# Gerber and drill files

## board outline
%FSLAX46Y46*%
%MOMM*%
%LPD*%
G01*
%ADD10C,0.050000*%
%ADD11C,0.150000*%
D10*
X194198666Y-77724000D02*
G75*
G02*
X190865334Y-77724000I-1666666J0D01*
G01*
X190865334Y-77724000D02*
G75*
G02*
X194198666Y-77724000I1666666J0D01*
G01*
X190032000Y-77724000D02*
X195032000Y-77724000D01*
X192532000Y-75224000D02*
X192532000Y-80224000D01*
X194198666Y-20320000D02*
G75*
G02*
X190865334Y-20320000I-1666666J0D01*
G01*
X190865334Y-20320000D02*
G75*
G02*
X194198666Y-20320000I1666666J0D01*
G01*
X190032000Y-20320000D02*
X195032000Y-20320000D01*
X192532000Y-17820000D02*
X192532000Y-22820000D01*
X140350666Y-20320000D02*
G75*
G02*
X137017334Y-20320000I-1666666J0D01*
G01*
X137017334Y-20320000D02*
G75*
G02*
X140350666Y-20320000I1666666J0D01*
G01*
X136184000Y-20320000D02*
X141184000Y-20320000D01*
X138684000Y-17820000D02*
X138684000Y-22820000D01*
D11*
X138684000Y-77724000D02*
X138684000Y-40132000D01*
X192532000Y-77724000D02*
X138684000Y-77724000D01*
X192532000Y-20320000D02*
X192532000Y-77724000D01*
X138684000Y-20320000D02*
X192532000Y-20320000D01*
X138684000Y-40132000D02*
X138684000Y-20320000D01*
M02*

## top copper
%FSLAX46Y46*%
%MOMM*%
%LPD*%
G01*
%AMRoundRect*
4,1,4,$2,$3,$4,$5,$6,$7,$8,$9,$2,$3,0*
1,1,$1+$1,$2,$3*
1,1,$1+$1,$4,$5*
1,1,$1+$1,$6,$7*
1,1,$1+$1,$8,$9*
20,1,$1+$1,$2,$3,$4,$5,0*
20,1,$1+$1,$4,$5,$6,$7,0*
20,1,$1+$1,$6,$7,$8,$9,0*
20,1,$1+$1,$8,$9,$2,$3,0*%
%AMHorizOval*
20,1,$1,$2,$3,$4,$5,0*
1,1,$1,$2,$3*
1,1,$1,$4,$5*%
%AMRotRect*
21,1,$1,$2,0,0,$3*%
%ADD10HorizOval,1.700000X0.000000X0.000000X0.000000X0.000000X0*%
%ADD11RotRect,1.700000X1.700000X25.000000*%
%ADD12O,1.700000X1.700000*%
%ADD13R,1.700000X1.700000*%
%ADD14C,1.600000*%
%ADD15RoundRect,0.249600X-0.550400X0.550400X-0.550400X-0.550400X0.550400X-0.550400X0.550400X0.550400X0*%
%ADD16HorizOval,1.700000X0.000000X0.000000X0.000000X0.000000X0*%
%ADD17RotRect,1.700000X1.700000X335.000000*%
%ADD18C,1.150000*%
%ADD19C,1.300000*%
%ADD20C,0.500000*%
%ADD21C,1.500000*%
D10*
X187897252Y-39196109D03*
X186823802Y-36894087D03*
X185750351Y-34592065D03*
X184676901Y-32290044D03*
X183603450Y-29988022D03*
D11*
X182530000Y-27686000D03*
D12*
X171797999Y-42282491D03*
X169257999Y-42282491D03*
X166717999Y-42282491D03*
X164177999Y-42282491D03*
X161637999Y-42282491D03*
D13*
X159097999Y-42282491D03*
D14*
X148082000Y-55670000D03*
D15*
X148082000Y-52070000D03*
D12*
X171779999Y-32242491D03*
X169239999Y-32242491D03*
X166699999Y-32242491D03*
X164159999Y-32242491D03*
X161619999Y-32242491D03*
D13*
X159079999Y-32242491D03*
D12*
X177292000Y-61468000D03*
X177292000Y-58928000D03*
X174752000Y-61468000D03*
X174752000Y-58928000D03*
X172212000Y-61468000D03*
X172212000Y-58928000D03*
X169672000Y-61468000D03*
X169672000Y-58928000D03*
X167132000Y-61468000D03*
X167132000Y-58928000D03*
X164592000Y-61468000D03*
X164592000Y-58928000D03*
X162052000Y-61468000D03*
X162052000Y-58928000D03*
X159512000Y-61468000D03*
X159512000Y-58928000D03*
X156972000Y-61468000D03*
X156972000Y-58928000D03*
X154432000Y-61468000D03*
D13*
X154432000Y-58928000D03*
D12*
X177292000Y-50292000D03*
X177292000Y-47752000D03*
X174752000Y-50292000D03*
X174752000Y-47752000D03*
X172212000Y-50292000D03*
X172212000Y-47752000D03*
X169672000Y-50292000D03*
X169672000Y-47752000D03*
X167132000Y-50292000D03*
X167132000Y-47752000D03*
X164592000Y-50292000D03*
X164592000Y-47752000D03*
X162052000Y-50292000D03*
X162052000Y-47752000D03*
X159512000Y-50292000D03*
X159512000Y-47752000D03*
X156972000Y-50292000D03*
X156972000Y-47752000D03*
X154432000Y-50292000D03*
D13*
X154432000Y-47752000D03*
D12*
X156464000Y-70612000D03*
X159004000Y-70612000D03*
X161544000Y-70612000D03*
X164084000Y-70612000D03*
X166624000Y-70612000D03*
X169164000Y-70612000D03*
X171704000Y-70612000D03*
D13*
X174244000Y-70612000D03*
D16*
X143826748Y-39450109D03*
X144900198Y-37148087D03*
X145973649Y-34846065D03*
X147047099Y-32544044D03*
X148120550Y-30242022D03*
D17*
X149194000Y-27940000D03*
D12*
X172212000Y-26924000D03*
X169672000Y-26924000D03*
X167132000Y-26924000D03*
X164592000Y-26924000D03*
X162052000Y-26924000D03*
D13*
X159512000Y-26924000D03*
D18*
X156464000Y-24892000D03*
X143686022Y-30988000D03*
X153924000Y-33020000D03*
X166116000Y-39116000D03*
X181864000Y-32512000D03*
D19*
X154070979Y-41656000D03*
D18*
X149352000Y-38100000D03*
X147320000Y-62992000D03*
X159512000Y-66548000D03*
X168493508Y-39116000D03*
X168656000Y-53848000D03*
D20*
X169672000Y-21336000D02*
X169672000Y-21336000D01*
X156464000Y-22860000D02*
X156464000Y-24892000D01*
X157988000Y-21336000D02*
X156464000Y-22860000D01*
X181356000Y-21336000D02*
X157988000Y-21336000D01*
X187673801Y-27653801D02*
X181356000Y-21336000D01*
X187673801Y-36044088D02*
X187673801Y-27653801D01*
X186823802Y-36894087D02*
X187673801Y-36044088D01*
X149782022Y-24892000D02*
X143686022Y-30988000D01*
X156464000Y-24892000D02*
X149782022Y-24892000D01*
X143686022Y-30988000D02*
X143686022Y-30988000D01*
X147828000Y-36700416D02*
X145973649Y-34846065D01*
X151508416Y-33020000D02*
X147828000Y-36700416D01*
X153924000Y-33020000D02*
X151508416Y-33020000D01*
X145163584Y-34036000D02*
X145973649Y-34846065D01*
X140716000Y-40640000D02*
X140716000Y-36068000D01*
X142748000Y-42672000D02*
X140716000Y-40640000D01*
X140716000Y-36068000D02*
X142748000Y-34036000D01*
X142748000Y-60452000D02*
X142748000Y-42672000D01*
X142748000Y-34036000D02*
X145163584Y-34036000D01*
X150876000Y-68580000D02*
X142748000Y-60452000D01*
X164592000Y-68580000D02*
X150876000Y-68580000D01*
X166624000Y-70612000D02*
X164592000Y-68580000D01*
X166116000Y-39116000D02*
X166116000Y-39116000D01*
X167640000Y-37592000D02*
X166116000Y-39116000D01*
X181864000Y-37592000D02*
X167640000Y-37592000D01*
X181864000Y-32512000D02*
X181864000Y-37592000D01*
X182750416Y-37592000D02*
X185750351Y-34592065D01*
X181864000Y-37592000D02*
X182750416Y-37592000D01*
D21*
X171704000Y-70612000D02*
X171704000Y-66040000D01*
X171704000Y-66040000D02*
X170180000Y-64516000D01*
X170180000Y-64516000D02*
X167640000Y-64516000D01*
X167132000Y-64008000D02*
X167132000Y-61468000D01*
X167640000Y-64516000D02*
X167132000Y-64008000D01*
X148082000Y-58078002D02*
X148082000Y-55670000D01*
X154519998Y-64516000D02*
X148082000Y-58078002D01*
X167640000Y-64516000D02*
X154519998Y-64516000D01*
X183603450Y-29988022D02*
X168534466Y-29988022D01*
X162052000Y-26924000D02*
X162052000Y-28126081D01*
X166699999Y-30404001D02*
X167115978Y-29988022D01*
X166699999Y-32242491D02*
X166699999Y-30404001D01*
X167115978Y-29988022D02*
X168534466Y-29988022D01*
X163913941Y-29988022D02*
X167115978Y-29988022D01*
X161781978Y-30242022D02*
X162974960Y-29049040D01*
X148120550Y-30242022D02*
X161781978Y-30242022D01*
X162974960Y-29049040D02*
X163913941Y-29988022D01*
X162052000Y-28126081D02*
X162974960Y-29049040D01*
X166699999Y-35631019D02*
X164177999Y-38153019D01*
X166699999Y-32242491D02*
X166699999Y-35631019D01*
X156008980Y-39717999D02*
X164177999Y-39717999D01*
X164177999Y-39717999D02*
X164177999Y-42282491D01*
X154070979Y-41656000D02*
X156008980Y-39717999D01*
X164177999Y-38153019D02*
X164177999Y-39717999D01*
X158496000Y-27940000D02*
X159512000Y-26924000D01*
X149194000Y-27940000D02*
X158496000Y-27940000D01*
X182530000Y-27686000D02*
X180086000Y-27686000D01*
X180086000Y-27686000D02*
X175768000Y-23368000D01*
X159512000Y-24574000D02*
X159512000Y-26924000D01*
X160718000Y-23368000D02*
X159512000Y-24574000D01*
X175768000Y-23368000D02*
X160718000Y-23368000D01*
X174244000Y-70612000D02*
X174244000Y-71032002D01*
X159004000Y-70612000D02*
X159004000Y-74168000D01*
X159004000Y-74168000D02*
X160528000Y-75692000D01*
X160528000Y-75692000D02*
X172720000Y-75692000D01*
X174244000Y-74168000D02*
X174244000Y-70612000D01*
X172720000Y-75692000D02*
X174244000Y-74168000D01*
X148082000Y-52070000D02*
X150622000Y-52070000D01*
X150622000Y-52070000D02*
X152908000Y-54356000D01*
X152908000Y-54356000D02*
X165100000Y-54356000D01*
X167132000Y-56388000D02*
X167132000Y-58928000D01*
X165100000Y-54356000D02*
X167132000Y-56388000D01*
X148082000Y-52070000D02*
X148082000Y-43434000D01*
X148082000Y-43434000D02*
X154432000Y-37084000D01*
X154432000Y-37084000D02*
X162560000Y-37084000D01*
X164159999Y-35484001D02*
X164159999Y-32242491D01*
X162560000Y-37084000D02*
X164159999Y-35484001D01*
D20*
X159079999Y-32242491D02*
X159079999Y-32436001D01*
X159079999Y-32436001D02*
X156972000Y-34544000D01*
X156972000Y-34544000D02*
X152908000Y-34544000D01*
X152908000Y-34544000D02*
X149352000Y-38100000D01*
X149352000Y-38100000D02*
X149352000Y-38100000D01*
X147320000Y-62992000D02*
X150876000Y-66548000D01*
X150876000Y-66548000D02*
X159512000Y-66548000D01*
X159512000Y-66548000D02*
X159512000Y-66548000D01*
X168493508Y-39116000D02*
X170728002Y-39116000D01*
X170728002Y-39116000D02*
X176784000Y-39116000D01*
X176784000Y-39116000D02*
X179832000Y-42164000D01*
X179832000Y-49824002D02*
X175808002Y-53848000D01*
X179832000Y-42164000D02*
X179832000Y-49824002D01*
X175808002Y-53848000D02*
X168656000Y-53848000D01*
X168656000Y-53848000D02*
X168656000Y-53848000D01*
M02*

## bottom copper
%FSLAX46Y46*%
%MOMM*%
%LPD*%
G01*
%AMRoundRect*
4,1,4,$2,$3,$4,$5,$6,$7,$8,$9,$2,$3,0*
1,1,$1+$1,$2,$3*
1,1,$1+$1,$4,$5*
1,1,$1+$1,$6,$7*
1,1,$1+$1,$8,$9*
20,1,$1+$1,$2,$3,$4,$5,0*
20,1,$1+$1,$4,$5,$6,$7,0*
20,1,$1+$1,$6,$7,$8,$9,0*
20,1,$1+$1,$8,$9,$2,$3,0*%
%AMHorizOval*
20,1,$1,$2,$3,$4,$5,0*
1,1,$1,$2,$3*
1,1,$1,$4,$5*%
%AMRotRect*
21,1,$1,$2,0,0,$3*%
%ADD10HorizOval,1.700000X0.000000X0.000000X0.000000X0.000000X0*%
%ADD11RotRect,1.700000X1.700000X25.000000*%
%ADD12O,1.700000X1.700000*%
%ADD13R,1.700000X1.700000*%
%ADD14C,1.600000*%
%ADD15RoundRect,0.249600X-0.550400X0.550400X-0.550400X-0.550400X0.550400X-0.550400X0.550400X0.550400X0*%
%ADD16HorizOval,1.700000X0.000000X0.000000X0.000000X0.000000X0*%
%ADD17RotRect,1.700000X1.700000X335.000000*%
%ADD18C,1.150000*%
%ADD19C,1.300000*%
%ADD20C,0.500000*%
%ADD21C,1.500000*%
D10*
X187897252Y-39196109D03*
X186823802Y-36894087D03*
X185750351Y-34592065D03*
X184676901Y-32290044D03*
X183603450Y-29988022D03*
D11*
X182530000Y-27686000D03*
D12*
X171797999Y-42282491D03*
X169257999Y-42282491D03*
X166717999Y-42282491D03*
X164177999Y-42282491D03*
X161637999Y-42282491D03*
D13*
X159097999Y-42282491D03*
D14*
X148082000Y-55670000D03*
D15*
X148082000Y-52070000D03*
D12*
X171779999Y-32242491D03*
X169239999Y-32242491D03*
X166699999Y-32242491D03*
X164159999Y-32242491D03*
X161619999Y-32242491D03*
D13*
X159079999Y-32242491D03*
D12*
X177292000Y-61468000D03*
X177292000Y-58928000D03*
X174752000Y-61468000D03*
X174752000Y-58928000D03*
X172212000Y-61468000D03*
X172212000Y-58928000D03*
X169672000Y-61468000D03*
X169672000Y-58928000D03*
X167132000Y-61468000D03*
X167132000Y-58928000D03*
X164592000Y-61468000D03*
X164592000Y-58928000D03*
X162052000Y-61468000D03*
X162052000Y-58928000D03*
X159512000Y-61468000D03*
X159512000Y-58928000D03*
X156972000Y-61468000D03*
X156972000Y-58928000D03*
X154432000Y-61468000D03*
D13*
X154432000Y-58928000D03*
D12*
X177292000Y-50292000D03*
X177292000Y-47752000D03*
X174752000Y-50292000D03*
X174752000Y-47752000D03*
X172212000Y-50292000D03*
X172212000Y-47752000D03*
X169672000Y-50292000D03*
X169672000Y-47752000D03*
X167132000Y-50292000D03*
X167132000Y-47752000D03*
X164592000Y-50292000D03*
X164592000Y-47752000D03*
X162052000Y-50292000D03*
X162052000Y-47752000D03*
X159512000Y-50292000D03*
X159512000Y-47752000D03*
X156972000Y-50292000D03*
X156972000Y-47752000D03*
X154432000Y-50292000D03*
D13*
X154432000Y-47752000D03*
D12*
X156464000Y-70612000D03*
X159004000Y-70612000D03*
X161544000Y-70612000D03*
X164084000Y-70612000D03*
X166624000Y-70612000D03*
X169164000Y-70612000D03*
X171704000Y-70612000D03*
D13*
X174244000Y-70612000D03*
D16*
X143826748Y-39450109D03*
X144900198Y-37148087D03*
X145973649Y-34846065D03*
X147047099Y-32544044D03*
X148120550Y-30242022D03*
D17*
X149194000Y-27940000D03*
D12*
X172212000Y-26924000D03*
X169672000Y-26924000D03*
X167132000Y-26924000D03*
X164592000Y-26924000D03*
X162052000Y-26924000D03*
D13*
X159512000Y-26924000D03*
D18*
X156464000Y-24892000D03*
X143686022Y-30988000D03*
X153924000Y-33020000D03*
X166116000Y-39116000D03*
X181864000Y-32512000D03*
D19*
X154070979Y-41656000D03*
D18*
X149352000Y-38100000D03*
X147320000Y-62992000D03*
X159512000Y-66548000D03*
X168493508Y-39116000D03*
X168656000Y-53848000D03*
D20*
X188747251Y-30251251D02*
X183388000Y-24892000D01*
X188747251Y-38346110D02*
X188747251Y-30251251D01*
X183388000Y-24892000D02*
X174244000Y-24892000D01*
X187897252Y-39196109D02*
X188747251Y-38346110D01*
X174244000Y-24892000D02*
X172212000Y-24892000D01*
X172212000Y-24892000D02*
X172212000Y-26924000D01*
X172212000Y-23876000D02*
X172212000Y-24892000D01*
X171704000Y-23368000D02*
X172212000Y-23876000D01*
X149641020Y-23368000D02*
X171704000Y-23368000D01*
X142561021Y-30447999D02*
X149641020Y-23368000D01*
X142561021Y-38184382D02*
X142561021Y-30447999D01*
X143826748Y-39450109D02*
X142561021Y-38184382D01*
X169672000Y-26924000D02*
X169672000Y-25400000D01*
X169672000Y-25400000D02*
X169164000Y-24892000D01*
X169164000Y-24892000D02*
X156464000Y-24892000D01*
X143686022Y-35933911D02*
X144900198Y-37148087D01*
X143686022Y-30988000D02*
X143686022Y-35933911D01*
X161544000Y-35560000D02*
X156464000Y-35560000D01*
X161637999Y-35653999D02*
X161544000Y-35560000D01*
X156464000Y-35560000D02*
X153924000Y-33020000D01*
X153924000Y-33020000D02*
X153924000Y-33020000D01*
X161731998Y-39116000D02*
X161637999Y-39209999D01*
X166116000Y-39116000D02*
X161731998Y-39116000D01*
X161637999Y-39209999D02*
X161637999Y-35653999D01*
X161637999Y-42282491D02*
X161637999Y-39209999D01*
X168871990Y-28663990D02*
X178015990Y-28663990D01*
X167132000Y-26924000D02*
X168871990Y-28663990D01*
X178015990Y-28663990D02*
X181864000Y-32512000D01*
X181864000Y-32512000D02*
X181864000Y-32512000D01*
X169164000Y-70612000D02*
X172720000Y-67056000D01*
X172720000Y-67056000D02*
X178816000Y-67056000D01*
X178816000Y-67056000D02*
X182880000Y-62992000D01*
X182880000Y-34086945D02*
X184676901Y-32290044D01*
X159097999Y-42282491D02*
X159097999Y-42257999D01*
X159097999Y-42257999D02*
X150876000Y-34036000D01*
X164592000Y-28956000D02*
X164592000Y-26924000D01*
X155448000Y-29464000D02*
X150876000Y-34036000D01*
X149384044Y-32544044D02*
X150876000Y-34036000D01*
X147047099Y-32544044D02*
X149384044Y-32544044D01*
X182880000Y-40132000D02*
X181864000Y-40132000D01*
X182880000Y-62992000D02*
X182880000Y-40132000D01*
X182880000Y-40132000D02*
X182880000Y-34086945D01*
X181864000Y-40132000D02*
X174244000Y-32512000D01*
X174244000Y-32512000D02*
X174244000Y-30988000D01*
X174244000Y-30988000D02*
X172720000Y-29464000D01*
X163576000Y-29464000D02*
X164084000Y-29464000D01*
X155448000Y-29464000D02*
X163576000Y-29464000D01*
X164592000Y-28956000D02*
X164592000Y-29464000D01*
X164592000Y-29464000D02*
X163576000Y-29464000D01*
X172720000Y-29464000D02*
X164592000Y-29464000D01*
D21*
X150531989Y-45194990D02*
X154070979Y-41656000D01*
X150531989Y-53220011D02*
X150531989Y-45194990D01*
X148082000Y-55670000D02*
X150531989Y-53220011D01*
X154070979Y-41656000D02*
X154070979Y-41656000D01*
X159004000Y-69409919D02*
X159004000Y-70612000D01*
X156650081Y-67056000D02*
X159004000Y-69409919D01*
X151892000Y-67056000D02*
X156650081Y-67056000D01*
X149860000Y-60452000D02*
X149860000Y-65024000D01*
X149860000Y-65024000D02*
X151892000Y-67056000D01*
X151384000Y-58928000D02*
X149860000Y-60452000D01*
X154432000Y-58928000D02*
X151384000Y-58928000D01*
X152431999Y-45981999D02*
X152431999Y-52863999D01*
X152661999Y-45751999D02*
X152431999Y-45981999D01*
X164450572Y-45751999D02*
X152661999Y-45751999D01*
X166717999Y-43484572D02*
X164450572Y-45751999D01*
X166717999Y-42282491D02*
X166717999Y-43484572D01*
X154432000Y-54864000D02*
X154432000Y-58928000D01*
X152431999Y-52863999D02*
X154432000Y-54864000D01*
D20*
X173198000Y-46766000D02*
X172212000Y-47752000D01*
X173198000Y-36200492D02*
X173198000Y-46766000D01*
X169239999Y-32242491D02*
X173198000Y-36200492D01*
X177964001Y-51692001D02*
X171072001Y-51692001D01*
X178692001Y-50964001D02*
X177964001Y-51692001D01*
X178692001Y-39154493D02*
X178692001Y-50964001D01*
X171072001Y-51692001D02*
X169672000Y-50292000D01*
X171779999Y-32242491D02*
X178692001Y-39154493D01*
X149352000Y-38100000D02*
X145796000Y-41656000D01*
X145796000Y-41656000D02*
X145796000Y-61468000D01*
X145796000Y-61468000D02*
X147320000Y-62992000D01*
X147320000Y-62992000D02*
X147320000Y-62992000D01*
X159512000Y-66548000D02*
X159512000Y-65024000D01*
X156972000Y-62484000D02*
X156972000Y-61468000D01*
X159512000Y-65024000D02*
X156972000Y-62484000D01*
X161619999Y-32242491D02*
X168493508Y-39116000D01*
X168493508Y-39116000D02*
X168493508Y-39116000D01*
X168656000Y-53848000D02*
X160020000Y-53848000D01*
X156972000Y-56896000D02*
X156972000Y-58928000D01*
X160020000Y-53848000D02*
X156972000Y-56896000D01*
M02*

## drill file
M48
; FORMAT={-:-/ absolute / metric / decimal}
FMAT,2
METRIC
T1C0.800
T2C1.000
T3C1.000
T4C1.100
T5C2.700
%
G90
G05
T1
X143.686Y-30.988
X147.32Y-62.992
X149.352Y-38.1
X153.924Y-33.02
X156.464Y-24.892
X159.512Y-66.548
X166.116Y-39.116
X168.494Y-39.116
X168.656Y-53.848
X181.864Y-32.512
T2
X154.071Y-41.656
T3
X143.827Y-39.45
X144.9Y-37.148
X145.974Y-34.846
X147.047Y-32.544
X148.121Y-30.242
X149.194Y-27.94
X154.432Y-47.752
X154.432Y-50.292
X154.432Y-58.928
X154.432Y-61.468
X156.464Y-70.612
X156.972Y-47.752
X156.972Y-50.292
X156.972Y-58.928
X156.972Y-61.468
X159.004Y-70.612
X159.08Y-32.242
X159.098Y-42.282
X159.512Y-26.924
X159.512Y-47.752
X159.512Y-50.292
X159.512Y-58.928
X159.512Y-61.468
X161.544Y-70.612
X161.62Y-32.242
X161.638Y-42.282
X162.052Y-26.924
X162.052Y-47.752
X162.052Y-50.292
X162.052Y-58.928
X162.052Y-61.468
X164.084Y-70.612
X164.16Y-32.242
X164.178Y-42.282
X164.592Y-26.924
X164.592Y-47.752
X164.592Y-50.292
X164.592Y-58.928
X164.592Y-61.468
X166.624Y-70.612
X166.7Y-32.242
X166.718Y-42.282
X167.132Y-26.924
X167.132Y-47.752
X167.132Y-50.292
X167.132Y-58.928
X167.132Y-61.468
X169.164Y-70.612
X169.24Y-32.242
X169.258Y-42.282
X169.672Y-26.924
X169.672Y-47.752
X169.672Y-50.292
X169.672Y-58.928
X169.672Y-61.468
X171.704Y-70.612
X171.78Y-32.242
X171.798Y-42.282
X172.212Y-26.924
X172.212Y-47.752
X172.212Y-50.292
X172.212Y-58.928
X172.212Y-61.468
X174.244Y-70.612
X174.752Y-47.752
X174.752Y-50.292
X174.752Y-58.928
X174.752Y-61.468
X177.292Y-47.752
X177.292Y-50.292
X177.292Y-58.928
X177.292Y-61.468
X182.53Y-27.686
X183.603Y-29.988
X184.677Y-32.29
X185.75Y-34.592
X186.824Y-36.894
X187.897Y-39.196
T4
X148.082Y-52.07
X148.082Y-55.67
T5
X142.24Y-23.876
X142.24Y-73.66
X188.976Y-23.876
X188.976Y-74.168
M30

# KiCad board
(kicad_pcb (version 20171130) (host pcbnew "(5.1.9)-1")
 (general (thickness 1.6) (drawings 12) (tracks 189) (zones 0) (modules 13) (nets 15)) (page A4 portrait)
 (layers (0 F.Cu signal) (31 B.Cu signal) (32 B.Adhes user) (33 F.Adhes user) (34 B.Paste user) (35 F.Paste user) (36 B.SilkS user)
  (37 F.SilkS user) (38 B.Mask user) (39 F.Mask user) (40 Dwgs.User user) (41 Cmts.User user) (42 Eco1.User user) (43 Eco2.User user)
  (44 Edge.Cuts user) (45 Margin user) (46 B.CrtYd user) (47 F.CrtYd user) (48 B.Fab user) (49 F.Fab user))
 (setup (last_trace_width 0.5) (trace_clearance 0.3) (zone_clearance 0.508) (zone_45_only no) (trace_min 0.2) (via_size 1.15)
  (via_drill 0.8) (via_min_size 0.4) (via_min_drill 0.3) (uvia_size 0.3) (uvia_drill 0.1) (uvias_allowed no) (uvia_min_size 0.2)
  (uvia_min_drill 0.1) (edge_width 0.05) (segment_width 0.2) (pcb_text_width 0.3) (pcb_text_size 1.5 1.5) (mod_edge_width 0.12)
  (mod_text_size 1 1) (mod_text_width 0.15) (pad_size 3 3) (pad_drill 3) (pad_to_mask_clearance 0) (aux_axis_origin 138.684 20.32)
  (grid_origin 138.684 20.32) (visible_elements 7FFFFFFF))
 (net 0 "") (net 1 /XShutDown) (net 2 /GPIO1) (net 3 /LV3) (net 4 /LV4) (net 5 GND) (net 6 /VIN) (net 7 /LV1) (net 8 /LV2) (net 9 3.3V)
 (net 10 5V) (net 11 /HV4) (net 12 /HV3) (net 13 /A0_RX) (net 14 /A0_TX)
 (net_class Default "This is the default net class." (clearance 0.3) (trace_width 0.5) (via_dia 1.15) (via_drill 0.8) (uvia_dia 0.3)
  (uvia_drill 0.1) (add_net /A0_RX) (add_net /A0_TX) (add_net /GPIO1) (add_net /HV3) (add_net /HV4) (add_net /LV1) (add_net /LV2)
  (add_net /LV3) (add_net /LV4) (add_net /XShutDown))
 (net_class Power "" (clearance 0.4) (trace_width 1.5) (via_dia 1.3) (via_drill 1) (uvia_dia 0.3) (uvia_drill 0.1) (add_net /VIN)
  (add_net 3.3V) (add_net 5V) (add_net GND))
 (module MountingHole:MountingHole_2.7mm (layer F.Cu) (at 142.24 73.66 90)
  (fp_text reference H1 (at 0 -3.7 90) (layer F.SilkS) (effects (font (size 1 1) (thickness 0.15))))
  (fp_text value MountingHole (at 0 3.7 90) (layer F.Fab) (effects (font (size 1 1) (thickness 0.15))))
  (pad 1 np_thru_hole circle (at 0 0 90) (size 2.7 2.7) (drill 2.7) (layers *.Cu *.Mask)))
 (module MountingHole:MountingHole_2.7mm (layer F.Cu) (at 142.24 23.876 90)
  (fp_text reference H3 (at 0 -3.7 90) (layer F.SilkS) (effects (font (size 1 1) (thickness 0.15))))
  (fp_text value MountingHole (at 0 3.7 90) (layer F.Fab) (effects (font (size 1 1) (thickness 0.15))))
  (pad 1 np_thru_hole circle (at 0 0 90) (size 2.7 2.7) (drill 2.7) (layers *.Cu *.Mask)))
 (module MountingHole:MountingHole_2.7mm (layer F.Cu) (at 188.976 74.168)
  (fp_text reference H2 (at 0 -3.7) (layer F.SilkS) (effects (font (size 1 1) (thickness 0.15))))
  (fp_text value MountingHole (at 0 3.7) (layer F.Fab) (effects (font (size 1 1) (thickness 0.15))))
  (pad 1 np_thru_hole circle (at 0 0) (size 2.7 2.7) (drill 2.7) (layers *.Cu *.Mask)))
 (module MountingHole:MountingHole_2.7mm (layer F.Cu) (at 188.976 23.876 90)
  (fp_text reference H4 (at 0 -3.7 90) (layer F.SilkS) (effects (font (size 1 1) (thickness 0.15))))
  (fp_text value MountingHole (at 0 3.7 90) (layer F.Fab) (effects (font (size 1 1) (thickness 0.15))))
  (pad 1 np_thru_hole circle (at 0 0 90) (size 2.7 2.7) (drill 2.7) (layers *.Cu *.Mask)))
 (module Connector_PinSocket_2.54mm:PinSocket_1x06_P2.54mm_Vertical (layer F.Cu) (at 182.53 27.686 25)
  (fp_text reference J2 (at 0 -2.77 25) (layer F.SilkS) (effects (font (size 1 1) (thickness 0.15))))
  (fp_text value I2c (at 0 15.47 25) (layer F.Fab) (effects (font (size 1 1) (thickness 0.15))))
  (pad 6 thru_hole oval (at 0 12.7 25) (size 1.7 1.7) (drill 1) (layers *.Cu *.Mask) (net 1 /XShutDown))
  (pad 5 thru_hole oval (at 0 10.16 25) (size 1.7 1.7) (drill 1) (layers *.Cu *.Mask) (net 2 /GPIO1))
  (pad 4 thru_hole oval (at 0 7.62 25) (size 1.7 1.7) (drill 1) (layers *.Cu *.Mask) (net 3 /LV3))
  (pad 3 thru_hole oval (at 0 5.08 25) (size 1.7 1.7) (drill 1) (layers *.Cu *.Mask) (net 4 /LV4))
  (pad 2 thru_hole oval (at 0 2.54 25) (size 1.7 1.7) (drill 1) (layers *.Cu *.Mask) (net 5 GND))
  (pad 1 thru_hole rect (at 0 0 25) (size 1.7 1.7) (drill 1) (layers *.Cu *.Mask) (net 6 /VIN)))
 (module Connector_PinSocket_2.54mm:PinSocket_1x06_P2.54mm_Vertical (layer F.Cu) (at 159.097999 42.282491 90)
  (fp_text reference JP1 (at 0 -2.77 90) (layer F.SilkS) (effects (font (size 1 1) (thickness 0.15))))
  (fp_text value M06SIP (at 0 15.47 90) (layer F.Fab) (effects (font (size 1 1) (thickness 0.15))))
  (pad 6 thru_hole oval (at 0 12.7 90) (size 1.7 1.7) (drill 1) (layers *.Cu *.Mask) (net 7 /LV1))
  (pad 5 thru_hole oval (at 0 10.16 90) (size 1.7 1.7) (drill 1) (layers *.Cu *.Mask) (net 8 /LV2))
  (pad 4 thru_hole oval (at 0 7.62 90) (size 1.7 1.7) (drill 1) (layers *.Cu *.Mask) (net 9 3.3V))
  (pad 3 thru_hole oval (at 0 5.08 90) (size 1.7 1.7) (drill 1) (layers *.Cu *.Mask) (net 5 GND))
  (pad 2 thru_hole oval (at 0 2.54 90) (size 1.7 1.7) (drill 1) (layers *.Cu *.Mask) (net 3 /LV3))
  (pad 1 thru_hole rect (at 0 0 90) (size 1.7 1.7) (drill 1) (layers *.Cu *.Mask) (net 4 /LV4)))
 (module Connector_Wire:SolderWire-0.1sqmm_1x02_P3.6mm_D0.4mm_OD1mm (layer F.Cu) (at 148.082 52.07 270)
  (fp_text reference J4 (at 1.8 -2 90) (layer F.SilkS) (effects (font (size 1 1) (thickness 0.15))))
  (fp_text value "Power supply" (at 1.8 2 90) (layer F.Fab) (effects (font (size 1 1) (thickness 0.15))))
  (pad 2 thru_hole circle (at 3.6 0 270) (size 1.6 1.6) (drill 1.1) (layers *.Cu *.Mask) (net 5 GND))
  (pad 1 thru_hole roundrect (at 0 0 270) (size 1.6 1.6) (drill 1.1) (layers *.Cu *.Mask) (roundrect_rratio 0.156) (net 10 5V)))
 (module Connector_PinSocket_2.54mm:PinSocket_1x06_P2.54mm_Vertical (layer F.Cu) (at 159.079999 32.242491 90)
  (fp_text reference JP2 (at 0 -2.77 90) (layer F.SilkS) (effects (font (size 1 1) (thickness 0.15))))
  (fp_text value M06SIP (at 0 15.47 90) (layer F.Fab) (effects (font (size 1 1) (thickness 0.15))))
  (pad 6 thru_hole oval (at 0 12.7 90) (size 1.7 1.7) (drill 1) (layers *.Cu *.Mask) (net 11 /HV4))
  (pad 5 thru_hole oval (at 0 10.16 90) (size 1.7 1.7) (drill 1) (layers *.Cu *.Mask) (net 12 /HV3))
  (pad 4 thru_hole oval (at 0 7.62 90) (size 1.7 1.7) (drill 1) (layers *.Cu *.Mask) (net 5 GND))
  (pad 3 thru_hole oval (at 0 5.08 90) (size 1.7 1.7) (drill 1) (layers *.Cu *.Mask) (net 10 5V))
  (pad 2 thru_hole oval (at 0 2.54 90) (size 1.7 1.7) (drill 1) (layers *.Cu *.Mask) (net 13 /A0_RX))
  (pad 1 thru_hole rect (at 0 0 90) (size 1.7 1.7) (drill 1) (layers *.Cu *.Mask) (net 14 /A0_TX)))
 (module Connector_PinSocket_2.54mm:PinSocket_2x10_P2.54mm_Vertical (layer F.Cu) (at 154.432 58.928 90)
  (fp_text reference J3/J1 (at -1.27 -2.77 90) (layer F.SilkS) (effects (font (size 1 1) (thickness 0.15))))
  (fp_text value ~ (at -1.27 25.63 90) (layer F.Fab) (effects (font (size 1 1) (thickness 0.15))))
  (pad 20 thru_hole oval (at -2.54 22.86 90) (size 1.7 1.7) (drill 1) (layers *.Cu *.Mask))
  (pad 19 thru_hole oval (at 0 22.86 90) (size 1.7 1.7) (drill 1) (layers *.Cu *.Mask))
  (pad 18 thru_hole oval (at -2.54 20.32 90) (size 1.7 1.7) (drill 1) (layers *.Cu *.Mask))
  (pad 17 thru_hole oval (at 0 20.32 90) (size 1.7 1.7) (drill 1) (layers *.Cu *.Mask))
  (pad 16 thru_hole oval (at -2.54 17.78 90) (size 1.7 1.7) (drill 1) (layers *.Cu *.Mask))
  (pad 15 thru_hole oval (at 0 17.78 90) (size 1.7 1.7) (drill 1) (layers *.Cu *.Mask))
  (pad 14 thru_hole oval (at -2.54 15.24 90) (size 1.7 1.7) (drill 1) (layers *.Cu *.Mask))
  (pad 13 thru_hole oval (at 0 15.24 90) (size 1.7 1.7) (drill 1) (layers *.Cu *.Mask))
  (pad 12 thru_hole oval (at -2.54 12.7 90) (size 1.7 1.7) (drill 1) (layers *.Cu *.Mask) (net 5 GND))
  (pad 11 thru_hole oval (at 0 12.7 90) (size 1.7 1.7) (drill 1) (layers *.Cu *.Mask) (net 10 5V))
  (pad 10 thru_hole oval (at -2.54 10.16 90) (size 1.7 1.7) (drill 1) (layers *.Cu *.Mask))
  (pad 9 thru_hole oval (at 0 10.16 90) (size 1.7 1.7) (drill 1) (layers *.Cu *.Mask))
  (pad 8 thru_hole oval (at -2.54 7.62 90) (size 1.7 1.7) (drill 1) (layers *.Cu *.Mask))
  (pad 7 thru_hole oval (at 0 7.62 90) (size 1.7 1.7) (drill 1) (layers *.Cu *.Mask))
  (pad 6 thru_hole oval (at -2.54 5.08 90) (size 1.7 1.7) (drill 1) (layers *.Cu *.Mask))
  (pad 5 thru_hole oval (at 0 5.08 90) (size 1.7 1.7) (drill 1) (layers *.Cu *.Mask))
  (pad 4 thru_hole oval (at -2.54 2.54 90) (size 1.7 1.7) (drill 1) (layers *.Cu *.Mask) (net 14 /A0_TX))
  (pad 3 thru_hole oval (at 0 2.54 90) (size 1.7 1.7) (drill 1) (layers *.Cu *.Mask) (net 13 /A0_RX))
  (pad 2 thru_hole oval (at -2.54 0 90) (size 1.7 1.7) (drill 1) (layers *.Cu *.Mask))
  (pad 1 thru_hole rect (at 0 0 90) (size 1.7 1.7) (drill 1) (layers *.Cu *.Mask) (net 9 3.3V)))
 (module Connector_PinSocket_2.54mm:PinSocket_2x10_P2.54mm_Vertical (layer F.Cu) (at 154.432 47.752 90)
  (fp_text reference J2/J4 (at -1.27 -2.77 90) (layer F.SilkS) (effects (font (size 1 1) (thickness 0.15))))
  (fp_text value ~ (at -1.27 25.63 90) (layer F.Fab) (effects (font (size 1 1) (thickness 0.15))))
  (pad 20 thru_hole oval (at -2.54 22.86 90) (size 1.7 1.7) (drill 1) (layers *.Cu *.Mask))
  (pad 19 thru_hole oval (at 0 22.86 90) (size 1.7 1.7) (drill 1) (layers *.Cu *.Mask))
  (pad 18 thru_hole oval (at -2.54 20.32 90) (size 1.7 1.7) (drill 1) (layers *.Cu *.Mask))
  (pad 17 thru_hole oval (at 0 20.32 90) (size 1.7 1.7) (drill 1) (layers *.Cu *.Mask))
  (pad 16 thru_hole oval (at -2.54 17.78 90) (size 1.7 1.7) (drill 1) (layers *.Cu *.Mask))
  (pad 15 thru_hole oval (at 0 17.78 90) (size 1.7 1.7) (drill 1) (layers *.Cu *.Mask) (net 12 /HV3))
  (pad 14 thru_hole oval (at -2.54 15.24 90) (size 1.7 1.7) (drill 1) (layers *.Cu *.Mask) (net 11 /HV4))
  (pad 13 thru_hole oval (at 0 15.24 90) (size 1.7 1.7) (drill 1) (layers *.Cu *.Mask))
  (pad 12 thru_hole oval (at -2.54 12.7 90) (size 1.7 1.7) (drill 1) (layers *.Cu *.Mask))
  (pad 11 thru_hole oval (at 0 12.7 90) (size 1.7 1.7) (drill 1) (layers *.Cu *.Mask))
  (pad 10 thru_hole oval (at -2.54 10.16 90) (size 1.7 1.7) (drill 1) (layers *.Cu *.Mask))
  (pad 9 thru_hole oval (at 0 10.16 90) (size 1.7 1.7) (drill 1) (layers *.Cu *.Mask))
  (pad 8 thru_hole oval (at -2.54 7.62 90) (size 1.7 1.7) (drill 1) (layers *.Cu *.Mask))
  (pad 7 thru_hole oval (at 0 7.62 90) (size 1.7 1.7) (drill 1) (layers *.Cu *.Mask))
  (pad 6 thru_hole oval (at -2.54 5.08 90) (size 1.7 1.7) (drill 1) (layers *.Cu *.Mask))
  (pad 5 thru_hole oval (at 0 5.08 90) (size 1.7 1.7) (drill 1) (layers *.Cu *.Mask))
  (pad 4 thru_hole oval (at -2.54 2.54 90) (size 1.7 1.7) (drill 1) (layers *.Cu *.Mask))
  (pad 3 thru_hole oval (at 0 2.54 90) (size 1.7 1.7) (drill 1) (layers *.Cu *.Mask))
  (pad 2 thru_hole oval (at -2.54 0 90) (size 1.7 1.7) (drill 1) (layers *.Cu *.Mask))
  (pad 1 thru_hole rect (at 0 0 90) (size 1.7 1.7) (drill 1) (layers *.Cu *.Mask)))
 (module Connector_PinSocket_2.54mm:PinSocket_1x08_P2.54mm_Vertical (layer F.Cu) (at 174.244 70.612 270)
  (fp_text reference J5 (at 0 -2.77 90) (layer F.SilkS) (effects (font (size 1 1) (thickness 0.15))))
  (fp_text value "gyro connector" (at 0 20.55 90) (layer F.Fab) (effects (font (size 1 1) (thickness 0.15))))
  (pad 8 thru_hole oval (at 0 17.78 270) (size 1.7 1.7) (drill 1) (layers *.Cu *.Mask))
  (pad 7 thru_hole oval (at 0 15.24 270) (size 1.7 1.7) (drill 1) (layers *.Cu *.Mask) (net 9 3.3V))
  (pad 6 thru_hole oval (at 0 12.7 270) (size 1.7 1.7) (drill 1) (layers *.Cu *.Mask))
  (pad 5 thru_hole oval (at 0 10.16 270) (size 1.7 1.7) (drill 1) (layers *.Cu *.Mask))
  (pad 4 thru_hole oval (at 0 7.62 270) (size 1.7 1.7) (drill 1) (layers *.Cu *.Mask) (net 3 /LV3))
  (pad 3 thru_hole oval (at 0 5.08 270) (size 1.7 1.7) (drill 1) (layers *.Cu *.Mask) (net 4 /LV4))
  (pad 2 thru_hole oval (at 0 2.54 270) (size 1.7 1.7) (drill 1) (layers *.Cu *.Mask) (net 5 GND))
  (pad 1 thru_hole rect (at 0 0 270) (size 1.7 1.7) (drill 1) (layers *.Cu *.Mask) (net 9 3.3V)))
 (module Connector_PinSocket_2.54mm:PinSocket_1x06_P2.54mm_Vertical (layer F.Cu) (at 149.194 27.94 335)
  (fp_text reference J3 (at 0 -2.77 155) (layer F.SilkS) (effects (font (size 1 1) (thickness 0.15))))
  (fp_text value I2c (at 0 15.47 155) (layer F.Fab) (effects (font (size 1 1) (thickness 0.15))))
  (pad 6 thru_hole oval (at 0 12.7 335) (size 1.7 1.7) (drill 1) (layers *.Cu *.Mask) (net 1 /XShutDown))
  (pad 5 thru_hole oval (at 0 10.16 335) (size 1.7 1.7) (drill 1) (layers *.Cu *.Mask) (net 2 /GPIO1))
  (pad 4 thru_hole oval (at 0 7.62 335) (size 1.7 1.7) (drill 1) (layers *.Cu *.Mask) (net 3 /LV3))
  (pad 3 thru_hole oval (at 0 5.08 335) (size 1.7 1.7) (drill 1) (layers *.Cu *.Mask) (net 4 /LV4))
  (pad 2 thru_hole oval (at 0 2.54 335) (size 1.7 1.7) (drill 1) (layers *.Cu *.Mask) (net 5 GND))
  (pad 1 thru_hole rect (at 0 0 335) (size 1.7 1.7) (drill 1) (layers *.Cu *.Mask) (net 6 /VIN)))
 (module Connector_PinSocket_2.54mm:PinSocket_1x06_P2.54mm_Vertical (layer F.Cu) (at 159.512 26.924 90)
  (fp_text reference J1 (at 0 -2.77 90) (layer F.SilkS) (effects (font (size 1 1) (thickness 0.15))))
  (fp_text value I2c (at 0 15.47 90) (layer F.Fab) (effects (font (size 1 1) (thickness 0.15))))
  (pad 6 thru_hole oval (at 0 12.7 90) (size 1.7 1.7) (drill 1) (layers *.Cu *.Mask) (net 1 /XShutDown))
  (pad 5 thru_hole oval (at 0 10.16 90) (size 1.7 1.7) (drill 1) (layers *.Cu *.Mask) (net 2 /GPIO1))
  (pad 4 thru_hole oval (at 0 7.62 90) (size 1.7 1.7) (drill 1) (layers *.Cu *.Mask) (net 3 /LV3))
  (pad 3 thru_hole oval (at 0 5.08 90) (size 1.7 1.7) (drill 1) (layers *.Cu *.Mask) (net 4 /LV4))
  (pad 2 thru_hole oval (at 0 2.54 90) (size 1.7 1.7) (drill 1) (layers *.Cu *.Mask) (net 5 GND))
  (pad 1 thru_hole rect (at 0 0 90) (size 1.7 1.7) (drill 1) (layers *.Cu *.Mask) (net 6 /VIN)))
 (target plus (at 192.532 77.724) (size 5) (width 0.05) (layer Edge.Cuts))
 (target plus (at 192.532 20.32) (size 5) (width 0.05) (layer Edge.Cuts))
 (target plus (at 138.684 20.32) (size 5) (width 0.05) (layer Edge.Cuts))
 (gr_line (start 138.684 77.724) (end 138.684 40.132) (layer Edge.Cuts) (width 0.15))
 (gr_line (start 192.532 77.724) (end 138.684 77.724) (layer Edge.Cuts) (width 0.15))
 (gr_line (start 192.532 20.32) (end 192.532 77.724) (layer Edge.Cuts) (width 0.15))
 (gr_line (start 138.684 20.32) (end 192.532 20.32) (layer Edge.Cuts) (width 0.15))
 (gr_line (start 138.684 40.132) (end 138.684 20.32) (layer Edge.Cuts) (width 0.15))
 (segment (start 188.747251 30.251251) (end 183.388 24.892) (width 0.5) (layer B.Cu) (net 1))
 (segment (start 188.747251 38.34611) (end 188.747251 30.251251) (width 0.5) (layer B.Cu) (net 1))
 (segment (start 183.388 24.892) (end 174.244 24.892) (width 0.5) (layer B.Cu) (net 1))
 (segment (start 187.897252 39.196109) (end 188.747251 38.34611) (width 0.5) (layer B.Cu) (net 1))
 (segment (start 174.244 24.892) (end 172.212 24.892) (width 0.5) (layer B.Cu) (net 1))
 (segment (start 172.212 24.892) (end 172.212 26.924) (width 0.5) (layer B.Cu) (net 1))
 (segment (start 172.212 23.876) (end 172.212 24.892) (width 0.5) (layer B.Cu) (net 1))
 (segment (start 171.704 23.368) (end 172.212 23.876) (width 0.5) (layer B.Cu) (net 1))
 (segment (start 149.64102 23.368) (end 171.704 23.368) (width 0.5) (layer B.Cu) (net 1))
 (segment (start 142.561021 30.447999) (end 149.64102 23.368) (width 0.5) (layer B.Cu) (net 1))
 (segment (start 142.561021 38.184382) (end 142.561021 30.447999) (width 0.5) (layer B.Cu) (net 1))
 (segment (start 143.826748 39.450109) (end 142.561021 38.184382) (width 0.5) (layer B.Cu) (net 1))
 (segment (start 169.672 21.336) (end 169.672 21.336) (width 0.5) (layer F.Cu) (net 2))
 (via (at 156.464 24.892) (size 1.15) (drill 0.8) (layers F.Cu B.Cu) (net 2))
 (segment (start 169.672 26.924) (end 169.672 25.4) (width 0.5) (layer B.Cu) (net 2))
 (segment (start 169.672 25.4) (end 169.164 24.892) (width 0.5) (layer B.Cu) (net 2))
 (segment (start 169.164 24.892) (end 156.464 24.892) (width 0.5) (layer B.Cu) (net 2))
 (segment (start 156.464 22.86) (end 156.464 24.892) (width 0.5) (layer F.Cu) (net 2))
 (segment (start 157.988 21.336) (end 156.464 22.86) (width 0.5) (layer F.Cu) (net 2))
 (segment (start 181.356 21.336) (end 157.988 21.336) (width 0.5) (layer F.Cu) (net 2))
 (segment (start 187.673801 27.653801) (end 181.356 21.336) (width 0.5) (layer F.Cu) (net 2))
 (segment (start 187.673801 36.044088) (end 187.673801 27.653801) (width 0.5) (layer F.Cu) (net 2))
 (segment (start 186.823802 36.894087) (end 187.673801 36.044088) (width 0.5) (layer F.Cu) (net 2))
 (segment (start 149.782022 24.892) (end 143.686022 30.988) (width 0.5) (layer F.Cu) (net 2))
 (segment (start 156.464 24.892) (end 149.782022 24.892) (width 0.5) (layer F.Cu) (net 2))
 (segment (start 143.686022 30.988) (end 143.686022 30.988) (width 0.5) (layer F.Cu) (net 2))
 (via (at 143.686022 30.988) (size 1.15) (drill 0.8) (layers F.Cu B.Cu) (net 2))
 (segment (start 143.686022 35.933911) (end 144.900198 37.148087) (width 0.5) (layer B.Cu) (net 2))
 (segment (start 143.686022 30.988) (end 143.686022 35.933911) (width 0.5) (layer B.Cu) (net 2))
 (segment (start 147.828 36.700416) (end 145.973649 34.846065) (width 0.5) (layer F.Cu) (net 3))
 (segment (start 161.544 35.56) (end 156.464 35.56) (width 0.5) (layer B.Cu) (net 3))
 (segment (start 161.637999 35.653999) (end 161.544 35.56) (width 0.5) (layer B.Cu) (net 3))
 (segment (start 156.464 35.56) (end 153.924 33.02) (width 0.5) (layer B.Cu) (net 3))
 (segment (start 153.924 33.02) (end 153.924 33.02) (width 0.5) (layer B.Cu) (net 3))
 (via (at 153.924 33.02) (size 1.15) (drill 0.8) (layers F.Cu B.Cu) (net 3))
 (segment (start 151.508416 33.02) (end 147.828 36.700416) (width 0.5) (layer F.Cu) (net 3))
 (segment (start 153.924 33.02) (end 151.508416 33.02) (width 0.5) (layer F.Cu) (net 3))
 (segment (start 145.163584 34.036) (end 145.973649 34.846065) (width 0.5) (layer F.Cu) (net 3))
 (segment (start 140.716 40.64) (end 140.716 36.068) (width 0.5) (layer F.Cu) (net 3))
 (segment (start 142.748 42.672) (end 140.716 40.64) (width 0.5) (layer F.Cu) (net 3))
 (segment (start 140.716 36.068) (end 142.748 34.036) (width 0.5) (layer F.Cu) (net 3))
 (segment (start 142.748 60.452) (end 142.748 42.672) (width 0.5) (layer F.Cu) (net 3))
 (segment (start 142.748 34.036) (end 145.163584 34.036) (width 0.5) (layer F.Cu) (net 3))
 (segment (start 150.876 68.58) (end 142.748 60.452) (width 0.5) (layer F.Cu) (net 3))
 (segment (start 164.592 68.58) (end 150.876 68.58) (width 0.5) (layer F.Cu) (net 3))
 (segment (start 166.624 70.612) (end 164.592 68.58) (width 0.5) (layer F.Cu) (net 3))
 (segment (start 166.116 39.116) (end 166.116 39.116) (width 0.5) (layer F.Cu) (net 3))
 (via (at 166.116 39.116) (size 1.15) (drill 0.8) (layers F.Cu B.Cu) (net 3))
 (segment (start 161.731998 39.116) (end 161.637999 39.209999) (width 0.5) (layer B.Cu) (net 3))
 (segment (start 166.116 39.116) (end 161.731998 39.116) (width 0.5) (layer B.Cu) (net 3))
 (segment (start 161.637999 39.209999) (end 161.637999 35.653999) (width 0.5) (layer B.Cu) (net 3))
 (segment (start 161.637999 42.282491) (end 161.637999 39.209999) (width 0.5) (layer B.Cu) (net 3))
 (segment (start 168.87199 28.66399) (end 178.01599 28.66399) (width 0.5) (layer B.Cu) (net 3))
 (segment (start 167.132 26.924) (end 168.87199 28.66399) (width 0.5) (layer B.Cu) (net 3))
 (segment (start 178.01599 28.66399) (end 181.864 32.512) (width 0.5) (layer B.Cu) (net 3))
 (segment (start 181.864 32.512) (end 181.864 32.512) (width 0.5) (layer B.Cu) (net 3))
 (via (at 181.864 32.512) (size 1.15) (drill 0.8) (layers F.Cu B.Cu) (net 3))
 (segment (start 167.64 37.592) (end 166.116 39.116) (width 0.5) (layer F.Cu) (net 3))
 (segment (start 181.864 37.592) (end 167.64 37.592) (width 0.5) (layer F.Cu) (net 3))
 (segment (start 181.864 32.512) (end 181.864 37.592) (width 0.5) (layer F.Cu) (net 3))
 (segment (start 182.750416 37.592) (end 185.750351 34.592065) (width 0.5) (layer F.Cu) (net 3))
 (segment (start 181.864 37.592) (end 182.750416 37.592) (width 0.5) (layer F.Cu) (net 3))
 (segment (start 169.164 70.612) (end 172.72 67.056) (width 0.5) (layer B.Cu) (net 4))
 (segment (start 172.72 67.056) (end 178.816 67.056) (width 0.5) (layer B.Cu) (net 4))
 (segment (start 178.816 67.056) (end 182.88 62.992) (width 0.5) (layer B.Cu) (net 4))
 (segment (start 182.88 34.086945) (end 184.676901 32.290044) (width 0.5) (layer B.Cu) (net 4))
 (segment (start 159.097999 42.282491) (end 159.097999 42.257999) (width 0.5) (layer B.Cu) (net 4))
 (segment (start 159.097999 42.257999) (end 150.876 34.036) (width 0.5) (layer B.Cu) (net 4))
 (segment (start 164.592 28.956) (end 164.592 26.924) (width 0.5) (layer B.Cu) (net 4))
 (segment (start 155.448 29.464) (end 150.876 34.036) (width 0.5) (layer B.Cu) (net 4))
 (segment (start 149.384044 32.544044) (end 150.876 34.036) (width 0.5) (layer B.Cu) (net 4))
 (segment (start 147.047099 32.544044) (end 149.384044 32.544044) (width 0.5) (layer B.Cu) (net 4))
 (segment (start 182.88 40.132) (end 181.864 40.132) (width 0.5) (layer B.Cu) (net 4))
 (segment (start 182.88 62.992) (end 182.88 40.132) (width 0.5) (layer B.Cu) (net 4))
 (segment (start 182.88 40.132) (end 182.88 34.086945) (width 0.5) (layer B.Cu) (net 4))
 (segment (start 181.864 40.132) (end 174.244 32.512) (width 0.5) (layer B.Cu) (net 4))
 (segment (start 174.244 32.512) (end 174.244 30.988) (width 0.5) (layer B.Cu) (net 4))
 (segment (start 174.244 30.988) (end 172.72 29.464) (width 0.5) (layer B.Cu) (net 4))
 (segment (start 163.576 29.464) (end 164.084 29.464) (width 0.5) (layer B.Cu) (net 4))
 (segment (start 155.448 29.464) (end 163.576 29.464) (width 0.5) (layer B.Cu) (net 4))
 (segment (start 164.592 28.956) (end 164.592 29.464) (width 0.5) (layer B.Cu) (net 4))
 (segment (start 164.592 29.464) (end 163.576 29.464) (width 0.5) (layer B.Cu) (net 4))
 (segment (start 172.72 29.464) (end 164.592 29.464) (width 0.5) (layer B.Cu) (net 4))
 (segment (start 171.704 70.612) (end 171.704 66.04) (width 1.5) (layer F.Cu) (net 5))
 (segment (start 171.704 66.04) (end 170.18 64.516) (width 1.5) (layer F.Cu) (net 5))
 (segment (start 170.18 64.516) (end 167.64 64.516) (width 1.5) (layer F.Cu) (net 5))
 (segment (start 167.132 64.008) (end 167.132 61.468) (width 1.5) (layer F.Cu) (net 5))
 (segment (start 167.64 64.516) (end 167.132 64.008) (width 1.5) (layer F.Cu) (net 5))
 (segment (start 148.082 58.078002) (end 148.082 55.67) (width 1.5) (layer F.Cu) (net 5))
 (segment (start 154.519998 64.516) (end 148.082 58.078002) (width 1.5) (layer F.Cu) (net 5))
 (segment (start 167.64 64.516) (end 154.519998 64.516) (width 1.5) (layer F.Cu) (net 5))
 (segment (start 183.60345 29.988022) (end 168.534466 29.988022) (width 1.5) (layer F.Cu) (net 5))
 (segment (start 162.052 26.924) (end 162.052 28.126081) (width 1.5) (layer F.Cu) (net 5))
 (segment (start 166.699999 30.404001) (end 167.115978 29.988022) (width 1.5) (layer F.Cu) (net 5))
 (segment (start 166.699999 32.242491) (end 166.699999 30.404001) (width 1.5) (layer F.Cu) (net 5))
 (segment (start 167.115978 29.988022) (end 168.534466 29.988022) (width 1.5) (layer F.Cu) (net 5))
 (segment (start 163.913941 29.988022) (end 167.115978 29.988022) (width 1.5) (layer F.Cu) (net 5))
 (segment (start 161.781978 30.242022) (end 162.97496 29.04904) (width 1.5) (layer F.Cu) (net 5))
 (segment (start 148.12055 30.242022) (end 161.781978 30.242022) (width 1.5) (layer F.Cu) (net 5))
 (segment (start 162.97496 29.04904) (end 163.913941 29.988022) (width 1.5) (layer F.Cu) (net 5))
 (segment (start 162.052 28.126081) (end 162.97496 29.04904) (width 1.5) (layer F.Cu) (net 5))
 (segment (start 166.699999 35.631019) (end 164.177999 38.153019) (width 1.5) (layer F.Cu) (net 5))
 (segment (start 166.699999 32.242491) (end 166.699999 35.631019) (width 1.5) (layer F.Cu) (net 5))
 (segment (start 150.531989 45.19499) (end 154.070979 41.656) (width 1.5) (layer B.Cu) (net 5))
 (segment (start 150.531989 53.220011) (end 150.531989 45.19499) (width 1.5) (layer B.Cu) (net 5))
 (segment (start 148.082 55.67) (end 150.531989 53.220011) (width 1.5) (layer B.Cu) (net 5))
 (segment (start 154.070979 41.656) (end 154.070979 41.656) (width 1.5) (layer B.Cu) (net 5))
 (via (at 154.070979 41.656) (size 1.3) (drill 1) (layers F.Cu B.Cu) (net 5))
 (segment (start 156.00898 39.717999) (end 164.177999 39.717999) (width 1.5) (layer F.Cu) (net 5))
 (segment (start 164.177999 39.717999) (end 164.177999 42.282491) (width 1.5) (layer F.Cu) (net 5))
 (segment (start 154.070979 41.656) (end 156.00898 39.717999) (width 1.5) (layer F.Cu) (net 5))
 (segment (start 164.177999 38.153019) (end 164.177999 39.717999) (width 1.5) (layer F.Cu) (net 5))
 (segment (start 158.496 27.94) (end 159.512 26.924) (width 1.5) (layer F.Cu) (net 6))
 (segment (start 149.194 27.94) (end 158.496 27.94) (width 1.5) (layer F.Cu) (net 6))
 (segment (start 182.53 27.686) (end 180.086 27.686) (width 1.5) (layer F.Cu) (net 6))
 (segment (start 180.086 27.686) (end 175.768 23.368) (width 1.5) (layer F.Cu) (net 6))
 (segment (start 159.512 24.574) (end 159.512 26.924) (width 1.5) (layer F.Cu) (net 6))
 (segment (start 160.718 23.368) (end 159.512 24.574) (width 1.5) (layer F.Cu) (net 6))
 (segment (start 175.768 23.368) (end 160.718 23.368) (width 1.5) (layer F.Cu) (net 6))
 (segment (start 174.244 70.612) (end 174.244 71.032002) (width 1.5) (layer F.Cu) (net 9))
 (segment (start 159.004 70.612) (end 159.004 74.168) (width 1.5) (layer F.Cu) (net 9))
 (segment (start 159.004 74.168) (end 160.528 75.692) (width 1.5) (layer F.Cu) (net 9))
 (segment (start 160.528 75.692) (end 172.72 75.692) (width 1.5) (layer F.Cu) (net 9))
 (segment (start 174.244 74.168) (end 174.244 70.612) (width 1.5) (layer F.Cu) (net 9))
 (segment (start 172.72 75.692) (end 174.244 74.168) (width 1.5) (layer F.Cu) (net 9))
 (segment (start 159.004 69.409919) (end 159.004 70.612) (width 1.5) (layer B.Cu) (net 9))
 (segment (start 156.650081 67.056) (end 159.004 69.409919) (width 1.5) (layer B.Cu) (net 9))
 (segment (start 151.892 67.056) (end 156.650081 67.056) (width 1.5) (layer B.Cu) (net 9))
 (segment (start 149.86 60.452) (end 149.86 65.024) (width 1.5) (layer B.Cu) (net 9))
 (segment (start 149.86 65.024) (end 151.892 67.056) (width 1.5) (layer B.Cu) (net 9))
 (segment (start 151.384 58.928) (end 149.86 60.452) (width 1.5) (layer B.Cu) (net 9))
 (segment (start 154.432 58.928) (end 151.384 58.928) (width 1.5) (layer B.Cu) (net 9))
 (segment (start 152.431999 45.981999) (end 152.431999 52.863999) (width 1.5) (layer B.Cu) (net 9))
 (segment (start 152.661999 45.751999) (end 152.431999 45.981999) (width 1.5) (layer B.Cu) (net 9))
 (segment (start 164.450572 45.751999) (end 152.661999 45.751999) (width 1.5) (layer B.Cu) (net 9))
 (segment (start 166.717999 43.484572) (end 164.450572 45.751999) (width 1.5) (layer B.Cu) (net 9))
 (segment (start 166.717999 42.282491) (end 166.717999 43.484572) (width 1.5) (layer B.Cu) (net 9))
 (segment (start 154.432 54.864) (end 154.432 58.928) (width 1.5) (layer B.Cu) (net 9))
 (segment (start 152.431999 52.863999) (end 154.432 54.864) (width 1.5) (layer B.Cu) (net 9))
 (segment (start 173.198 46.766) (end 172.212 47.752) (width 0.5) (layer B.Cu) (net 12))
 (segment (start 173.198 36.200492) (end 173.198 46.766) (width 0.5) (layer B.Cu) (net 12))
 (segment (start 169.239999 32.242491) (end 173.198 36.200492) (width 0.5) (layer B.Cu) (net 12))
 (segment (start 177.964001 51.692001) (end 171.072001 51.692001) (width 0.5) (layer B.Cu) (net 11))
 (segment (start 178.692001 50.964001) (end 177.964001 51.692001) (width 0.5) (layer B.Cu) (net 11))
 (segment (start 178.692001 39.154493) (end 178.692001 50.964001) (width 0.5) (layer B.Cu) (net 11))
 (segment (start 171.072001 51.692001) (end 169.672 50.292) (width 0.5) (layer B.Cu) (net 11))
 (segment (start 171.779999 32.242491) (end 178.692001 39.154493) (width 0.5) (layer B.Cu) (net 11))
 (segment (start 148.082 52.07) (end 150.622 52.07) (width 1.5) (layer F.Cu) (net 10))
 (segment (start 150.622 52.07) (end 152.908 54.356) (width 1.5) (layer F.Cu) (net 10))
 (segment (start 152.908 54.356) (end 165.1 54.356) (width 1.5) (layer F.Cu) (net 10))
 (segment (start 167.132 56.388) (end 167.132 58.928) (width 1.5) (layer F.Cu) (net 10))
 (segment (start 165.1 54.356) (end 167.132 56.388) (width 1.5) (layer F.Cu) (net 10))
 (segment (start 148.082 52.07) (end 148.082 43.434) (width 1.5) (layer F.Cu) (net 10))
 (segment (start 148.082 43.434) (end 154.432 37.084) (width 1.5) (layer F.Cu) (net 10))
 (segment (start 154.432 37.084) (end 162.56 37.084) (width 1.5) (layer F.Cu) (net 10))
 (segment (start 164.159999 35.484001) (end 164.159999 32.242491) (width 1.5) (layer F.Cu) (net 10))
 (segment (start 162.56 37.084) (end 164.159999 35.484001) (width 1.5) (layer F.Cu) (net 10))
 (segment (start 159.079999 32.242491) (end 159.079999 32.436001) (width 0.5) (layer F.Cu) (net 14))
 (segment (start 159.079999 32.436001) (end 156.972 34.544) (width 0.5) (layer F.Cu) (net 14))
 (segment (start 156.972 34.544) (end 152.908 34.544) (width 0.5) (layer F.Cu) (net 14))
 (segment (start 152.908 34.544) (end 149.352 38.1) (width 0.5) (layer F.Cu) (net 14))
 (segment (start 149.352 38.1) (end 149.352 38.1) (width 0.5) (layer F.Cu) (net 14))
 (via (at 149.352 38.1) (size 1.15) (drill 0.8) (layers F.Cu B.Cu) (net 14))
 (segment (start 149.352 38.1) (end 145.796 41.656) (width 0.5) (layer B.Cu) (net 14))
 (segment (start 145.796 41.656) (end 145.796 61.468) (width 0.5) (layer B.Cu) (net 14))
 (segment (start 145.796 61.468) (end 147.32 62.992) (width 0.5) (layer B.Cu) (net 14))
 (segment (start 147.32 62.992) (end 147.32 62.992) (width 0.5) (layer B.Cu) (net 14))
 (via (at 147.32 62.992) (size 1.15) (drill 0.8) (layers F.Cu B.Cu) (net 14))
 (segment (start 147.32 62.992) (end 150.876 66.548) (width 0.5) (layer F.Cu) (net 14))
 (segment (start 150.876 66.548) (end 159.512 66.548) (width 0.5) (layer F.Cu) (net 14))
 (segment (start 159.512 66.548) (end 159.512 66.548) (width 0.5) (layer F.Cu) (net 14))
 (via (at 159.512 66.548) (size 1.15) (drill 0.8) (layers F.Cu B.Cu) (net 14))
 (segment (start 159.512 66.548) (end 159.512 65.024) (width 0.5) (layer B.Cu) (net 14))
 (segment (start 156.972 62.484) (end 156.972 61.468) (width 0.5) (layer B.Cu) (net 14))
 (segment (start 159.512 65.024) (end 156.972 62.484) (width 0.5) (layer B.Cu) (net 14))
 (segment (start 161.619999 32.242491) (end 168.493508 39.116) (width 0.5) (layer B.Cu) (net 13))
 (segment (start 168.493508 39.116) (end 168.493508 39.116) (width 0.5) (layer B.Cu) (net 13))
 (via (at 168.493508 39.116) (size 1.15) (drill 0.8) (layers F.Cu B.Cu) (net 13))
 (segment (start 168.493508 39.116) (end 170.728002 39.116) (width 0.5) (layer F.Cu) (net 13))
 (segment (start 170.728002 39.116) (end 176.784 39.116) (width 0.5) (layer F.Cu) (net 13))
 (segment (start 176.784 39.116) (end 179.832 42.164) (width 0.5) (layer F.Cu) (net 13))
 (segment (start 179.832 49.824002) (end 175.808002 53.848) (width 0.5) (layer F.Cu) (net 13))
 (segment (start 179.832 42.164) (end 179.832 49.824002) (width 0.5) (layer F.Cu) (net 13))
 (segment (start 175.808002 53.848) (end 168.656 53.848) (width 0.5) (layer F.Cu) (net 13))
 (segment (start 168.656 53.848) (end 168.656 53.848) (width 0.5) (layer F.Cu) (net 13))
 (via (at 168.656 53.848) (size 1.15) (drill 0.8) (layers F.Cu B.Cu) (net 13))
 (segment (start 168.656 53.848) (end 160.02 53.848) (width 0.5) (layer B.Cu) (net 13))
 (segment (start 156.972 56.896) (end 156.972 58.928) (width 0.5) (layer B.Cu) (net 13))
 (segment (start 160.02 53.848) (end 156.972 56.896) (width 0.5) (layer B.Cu) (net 13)))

